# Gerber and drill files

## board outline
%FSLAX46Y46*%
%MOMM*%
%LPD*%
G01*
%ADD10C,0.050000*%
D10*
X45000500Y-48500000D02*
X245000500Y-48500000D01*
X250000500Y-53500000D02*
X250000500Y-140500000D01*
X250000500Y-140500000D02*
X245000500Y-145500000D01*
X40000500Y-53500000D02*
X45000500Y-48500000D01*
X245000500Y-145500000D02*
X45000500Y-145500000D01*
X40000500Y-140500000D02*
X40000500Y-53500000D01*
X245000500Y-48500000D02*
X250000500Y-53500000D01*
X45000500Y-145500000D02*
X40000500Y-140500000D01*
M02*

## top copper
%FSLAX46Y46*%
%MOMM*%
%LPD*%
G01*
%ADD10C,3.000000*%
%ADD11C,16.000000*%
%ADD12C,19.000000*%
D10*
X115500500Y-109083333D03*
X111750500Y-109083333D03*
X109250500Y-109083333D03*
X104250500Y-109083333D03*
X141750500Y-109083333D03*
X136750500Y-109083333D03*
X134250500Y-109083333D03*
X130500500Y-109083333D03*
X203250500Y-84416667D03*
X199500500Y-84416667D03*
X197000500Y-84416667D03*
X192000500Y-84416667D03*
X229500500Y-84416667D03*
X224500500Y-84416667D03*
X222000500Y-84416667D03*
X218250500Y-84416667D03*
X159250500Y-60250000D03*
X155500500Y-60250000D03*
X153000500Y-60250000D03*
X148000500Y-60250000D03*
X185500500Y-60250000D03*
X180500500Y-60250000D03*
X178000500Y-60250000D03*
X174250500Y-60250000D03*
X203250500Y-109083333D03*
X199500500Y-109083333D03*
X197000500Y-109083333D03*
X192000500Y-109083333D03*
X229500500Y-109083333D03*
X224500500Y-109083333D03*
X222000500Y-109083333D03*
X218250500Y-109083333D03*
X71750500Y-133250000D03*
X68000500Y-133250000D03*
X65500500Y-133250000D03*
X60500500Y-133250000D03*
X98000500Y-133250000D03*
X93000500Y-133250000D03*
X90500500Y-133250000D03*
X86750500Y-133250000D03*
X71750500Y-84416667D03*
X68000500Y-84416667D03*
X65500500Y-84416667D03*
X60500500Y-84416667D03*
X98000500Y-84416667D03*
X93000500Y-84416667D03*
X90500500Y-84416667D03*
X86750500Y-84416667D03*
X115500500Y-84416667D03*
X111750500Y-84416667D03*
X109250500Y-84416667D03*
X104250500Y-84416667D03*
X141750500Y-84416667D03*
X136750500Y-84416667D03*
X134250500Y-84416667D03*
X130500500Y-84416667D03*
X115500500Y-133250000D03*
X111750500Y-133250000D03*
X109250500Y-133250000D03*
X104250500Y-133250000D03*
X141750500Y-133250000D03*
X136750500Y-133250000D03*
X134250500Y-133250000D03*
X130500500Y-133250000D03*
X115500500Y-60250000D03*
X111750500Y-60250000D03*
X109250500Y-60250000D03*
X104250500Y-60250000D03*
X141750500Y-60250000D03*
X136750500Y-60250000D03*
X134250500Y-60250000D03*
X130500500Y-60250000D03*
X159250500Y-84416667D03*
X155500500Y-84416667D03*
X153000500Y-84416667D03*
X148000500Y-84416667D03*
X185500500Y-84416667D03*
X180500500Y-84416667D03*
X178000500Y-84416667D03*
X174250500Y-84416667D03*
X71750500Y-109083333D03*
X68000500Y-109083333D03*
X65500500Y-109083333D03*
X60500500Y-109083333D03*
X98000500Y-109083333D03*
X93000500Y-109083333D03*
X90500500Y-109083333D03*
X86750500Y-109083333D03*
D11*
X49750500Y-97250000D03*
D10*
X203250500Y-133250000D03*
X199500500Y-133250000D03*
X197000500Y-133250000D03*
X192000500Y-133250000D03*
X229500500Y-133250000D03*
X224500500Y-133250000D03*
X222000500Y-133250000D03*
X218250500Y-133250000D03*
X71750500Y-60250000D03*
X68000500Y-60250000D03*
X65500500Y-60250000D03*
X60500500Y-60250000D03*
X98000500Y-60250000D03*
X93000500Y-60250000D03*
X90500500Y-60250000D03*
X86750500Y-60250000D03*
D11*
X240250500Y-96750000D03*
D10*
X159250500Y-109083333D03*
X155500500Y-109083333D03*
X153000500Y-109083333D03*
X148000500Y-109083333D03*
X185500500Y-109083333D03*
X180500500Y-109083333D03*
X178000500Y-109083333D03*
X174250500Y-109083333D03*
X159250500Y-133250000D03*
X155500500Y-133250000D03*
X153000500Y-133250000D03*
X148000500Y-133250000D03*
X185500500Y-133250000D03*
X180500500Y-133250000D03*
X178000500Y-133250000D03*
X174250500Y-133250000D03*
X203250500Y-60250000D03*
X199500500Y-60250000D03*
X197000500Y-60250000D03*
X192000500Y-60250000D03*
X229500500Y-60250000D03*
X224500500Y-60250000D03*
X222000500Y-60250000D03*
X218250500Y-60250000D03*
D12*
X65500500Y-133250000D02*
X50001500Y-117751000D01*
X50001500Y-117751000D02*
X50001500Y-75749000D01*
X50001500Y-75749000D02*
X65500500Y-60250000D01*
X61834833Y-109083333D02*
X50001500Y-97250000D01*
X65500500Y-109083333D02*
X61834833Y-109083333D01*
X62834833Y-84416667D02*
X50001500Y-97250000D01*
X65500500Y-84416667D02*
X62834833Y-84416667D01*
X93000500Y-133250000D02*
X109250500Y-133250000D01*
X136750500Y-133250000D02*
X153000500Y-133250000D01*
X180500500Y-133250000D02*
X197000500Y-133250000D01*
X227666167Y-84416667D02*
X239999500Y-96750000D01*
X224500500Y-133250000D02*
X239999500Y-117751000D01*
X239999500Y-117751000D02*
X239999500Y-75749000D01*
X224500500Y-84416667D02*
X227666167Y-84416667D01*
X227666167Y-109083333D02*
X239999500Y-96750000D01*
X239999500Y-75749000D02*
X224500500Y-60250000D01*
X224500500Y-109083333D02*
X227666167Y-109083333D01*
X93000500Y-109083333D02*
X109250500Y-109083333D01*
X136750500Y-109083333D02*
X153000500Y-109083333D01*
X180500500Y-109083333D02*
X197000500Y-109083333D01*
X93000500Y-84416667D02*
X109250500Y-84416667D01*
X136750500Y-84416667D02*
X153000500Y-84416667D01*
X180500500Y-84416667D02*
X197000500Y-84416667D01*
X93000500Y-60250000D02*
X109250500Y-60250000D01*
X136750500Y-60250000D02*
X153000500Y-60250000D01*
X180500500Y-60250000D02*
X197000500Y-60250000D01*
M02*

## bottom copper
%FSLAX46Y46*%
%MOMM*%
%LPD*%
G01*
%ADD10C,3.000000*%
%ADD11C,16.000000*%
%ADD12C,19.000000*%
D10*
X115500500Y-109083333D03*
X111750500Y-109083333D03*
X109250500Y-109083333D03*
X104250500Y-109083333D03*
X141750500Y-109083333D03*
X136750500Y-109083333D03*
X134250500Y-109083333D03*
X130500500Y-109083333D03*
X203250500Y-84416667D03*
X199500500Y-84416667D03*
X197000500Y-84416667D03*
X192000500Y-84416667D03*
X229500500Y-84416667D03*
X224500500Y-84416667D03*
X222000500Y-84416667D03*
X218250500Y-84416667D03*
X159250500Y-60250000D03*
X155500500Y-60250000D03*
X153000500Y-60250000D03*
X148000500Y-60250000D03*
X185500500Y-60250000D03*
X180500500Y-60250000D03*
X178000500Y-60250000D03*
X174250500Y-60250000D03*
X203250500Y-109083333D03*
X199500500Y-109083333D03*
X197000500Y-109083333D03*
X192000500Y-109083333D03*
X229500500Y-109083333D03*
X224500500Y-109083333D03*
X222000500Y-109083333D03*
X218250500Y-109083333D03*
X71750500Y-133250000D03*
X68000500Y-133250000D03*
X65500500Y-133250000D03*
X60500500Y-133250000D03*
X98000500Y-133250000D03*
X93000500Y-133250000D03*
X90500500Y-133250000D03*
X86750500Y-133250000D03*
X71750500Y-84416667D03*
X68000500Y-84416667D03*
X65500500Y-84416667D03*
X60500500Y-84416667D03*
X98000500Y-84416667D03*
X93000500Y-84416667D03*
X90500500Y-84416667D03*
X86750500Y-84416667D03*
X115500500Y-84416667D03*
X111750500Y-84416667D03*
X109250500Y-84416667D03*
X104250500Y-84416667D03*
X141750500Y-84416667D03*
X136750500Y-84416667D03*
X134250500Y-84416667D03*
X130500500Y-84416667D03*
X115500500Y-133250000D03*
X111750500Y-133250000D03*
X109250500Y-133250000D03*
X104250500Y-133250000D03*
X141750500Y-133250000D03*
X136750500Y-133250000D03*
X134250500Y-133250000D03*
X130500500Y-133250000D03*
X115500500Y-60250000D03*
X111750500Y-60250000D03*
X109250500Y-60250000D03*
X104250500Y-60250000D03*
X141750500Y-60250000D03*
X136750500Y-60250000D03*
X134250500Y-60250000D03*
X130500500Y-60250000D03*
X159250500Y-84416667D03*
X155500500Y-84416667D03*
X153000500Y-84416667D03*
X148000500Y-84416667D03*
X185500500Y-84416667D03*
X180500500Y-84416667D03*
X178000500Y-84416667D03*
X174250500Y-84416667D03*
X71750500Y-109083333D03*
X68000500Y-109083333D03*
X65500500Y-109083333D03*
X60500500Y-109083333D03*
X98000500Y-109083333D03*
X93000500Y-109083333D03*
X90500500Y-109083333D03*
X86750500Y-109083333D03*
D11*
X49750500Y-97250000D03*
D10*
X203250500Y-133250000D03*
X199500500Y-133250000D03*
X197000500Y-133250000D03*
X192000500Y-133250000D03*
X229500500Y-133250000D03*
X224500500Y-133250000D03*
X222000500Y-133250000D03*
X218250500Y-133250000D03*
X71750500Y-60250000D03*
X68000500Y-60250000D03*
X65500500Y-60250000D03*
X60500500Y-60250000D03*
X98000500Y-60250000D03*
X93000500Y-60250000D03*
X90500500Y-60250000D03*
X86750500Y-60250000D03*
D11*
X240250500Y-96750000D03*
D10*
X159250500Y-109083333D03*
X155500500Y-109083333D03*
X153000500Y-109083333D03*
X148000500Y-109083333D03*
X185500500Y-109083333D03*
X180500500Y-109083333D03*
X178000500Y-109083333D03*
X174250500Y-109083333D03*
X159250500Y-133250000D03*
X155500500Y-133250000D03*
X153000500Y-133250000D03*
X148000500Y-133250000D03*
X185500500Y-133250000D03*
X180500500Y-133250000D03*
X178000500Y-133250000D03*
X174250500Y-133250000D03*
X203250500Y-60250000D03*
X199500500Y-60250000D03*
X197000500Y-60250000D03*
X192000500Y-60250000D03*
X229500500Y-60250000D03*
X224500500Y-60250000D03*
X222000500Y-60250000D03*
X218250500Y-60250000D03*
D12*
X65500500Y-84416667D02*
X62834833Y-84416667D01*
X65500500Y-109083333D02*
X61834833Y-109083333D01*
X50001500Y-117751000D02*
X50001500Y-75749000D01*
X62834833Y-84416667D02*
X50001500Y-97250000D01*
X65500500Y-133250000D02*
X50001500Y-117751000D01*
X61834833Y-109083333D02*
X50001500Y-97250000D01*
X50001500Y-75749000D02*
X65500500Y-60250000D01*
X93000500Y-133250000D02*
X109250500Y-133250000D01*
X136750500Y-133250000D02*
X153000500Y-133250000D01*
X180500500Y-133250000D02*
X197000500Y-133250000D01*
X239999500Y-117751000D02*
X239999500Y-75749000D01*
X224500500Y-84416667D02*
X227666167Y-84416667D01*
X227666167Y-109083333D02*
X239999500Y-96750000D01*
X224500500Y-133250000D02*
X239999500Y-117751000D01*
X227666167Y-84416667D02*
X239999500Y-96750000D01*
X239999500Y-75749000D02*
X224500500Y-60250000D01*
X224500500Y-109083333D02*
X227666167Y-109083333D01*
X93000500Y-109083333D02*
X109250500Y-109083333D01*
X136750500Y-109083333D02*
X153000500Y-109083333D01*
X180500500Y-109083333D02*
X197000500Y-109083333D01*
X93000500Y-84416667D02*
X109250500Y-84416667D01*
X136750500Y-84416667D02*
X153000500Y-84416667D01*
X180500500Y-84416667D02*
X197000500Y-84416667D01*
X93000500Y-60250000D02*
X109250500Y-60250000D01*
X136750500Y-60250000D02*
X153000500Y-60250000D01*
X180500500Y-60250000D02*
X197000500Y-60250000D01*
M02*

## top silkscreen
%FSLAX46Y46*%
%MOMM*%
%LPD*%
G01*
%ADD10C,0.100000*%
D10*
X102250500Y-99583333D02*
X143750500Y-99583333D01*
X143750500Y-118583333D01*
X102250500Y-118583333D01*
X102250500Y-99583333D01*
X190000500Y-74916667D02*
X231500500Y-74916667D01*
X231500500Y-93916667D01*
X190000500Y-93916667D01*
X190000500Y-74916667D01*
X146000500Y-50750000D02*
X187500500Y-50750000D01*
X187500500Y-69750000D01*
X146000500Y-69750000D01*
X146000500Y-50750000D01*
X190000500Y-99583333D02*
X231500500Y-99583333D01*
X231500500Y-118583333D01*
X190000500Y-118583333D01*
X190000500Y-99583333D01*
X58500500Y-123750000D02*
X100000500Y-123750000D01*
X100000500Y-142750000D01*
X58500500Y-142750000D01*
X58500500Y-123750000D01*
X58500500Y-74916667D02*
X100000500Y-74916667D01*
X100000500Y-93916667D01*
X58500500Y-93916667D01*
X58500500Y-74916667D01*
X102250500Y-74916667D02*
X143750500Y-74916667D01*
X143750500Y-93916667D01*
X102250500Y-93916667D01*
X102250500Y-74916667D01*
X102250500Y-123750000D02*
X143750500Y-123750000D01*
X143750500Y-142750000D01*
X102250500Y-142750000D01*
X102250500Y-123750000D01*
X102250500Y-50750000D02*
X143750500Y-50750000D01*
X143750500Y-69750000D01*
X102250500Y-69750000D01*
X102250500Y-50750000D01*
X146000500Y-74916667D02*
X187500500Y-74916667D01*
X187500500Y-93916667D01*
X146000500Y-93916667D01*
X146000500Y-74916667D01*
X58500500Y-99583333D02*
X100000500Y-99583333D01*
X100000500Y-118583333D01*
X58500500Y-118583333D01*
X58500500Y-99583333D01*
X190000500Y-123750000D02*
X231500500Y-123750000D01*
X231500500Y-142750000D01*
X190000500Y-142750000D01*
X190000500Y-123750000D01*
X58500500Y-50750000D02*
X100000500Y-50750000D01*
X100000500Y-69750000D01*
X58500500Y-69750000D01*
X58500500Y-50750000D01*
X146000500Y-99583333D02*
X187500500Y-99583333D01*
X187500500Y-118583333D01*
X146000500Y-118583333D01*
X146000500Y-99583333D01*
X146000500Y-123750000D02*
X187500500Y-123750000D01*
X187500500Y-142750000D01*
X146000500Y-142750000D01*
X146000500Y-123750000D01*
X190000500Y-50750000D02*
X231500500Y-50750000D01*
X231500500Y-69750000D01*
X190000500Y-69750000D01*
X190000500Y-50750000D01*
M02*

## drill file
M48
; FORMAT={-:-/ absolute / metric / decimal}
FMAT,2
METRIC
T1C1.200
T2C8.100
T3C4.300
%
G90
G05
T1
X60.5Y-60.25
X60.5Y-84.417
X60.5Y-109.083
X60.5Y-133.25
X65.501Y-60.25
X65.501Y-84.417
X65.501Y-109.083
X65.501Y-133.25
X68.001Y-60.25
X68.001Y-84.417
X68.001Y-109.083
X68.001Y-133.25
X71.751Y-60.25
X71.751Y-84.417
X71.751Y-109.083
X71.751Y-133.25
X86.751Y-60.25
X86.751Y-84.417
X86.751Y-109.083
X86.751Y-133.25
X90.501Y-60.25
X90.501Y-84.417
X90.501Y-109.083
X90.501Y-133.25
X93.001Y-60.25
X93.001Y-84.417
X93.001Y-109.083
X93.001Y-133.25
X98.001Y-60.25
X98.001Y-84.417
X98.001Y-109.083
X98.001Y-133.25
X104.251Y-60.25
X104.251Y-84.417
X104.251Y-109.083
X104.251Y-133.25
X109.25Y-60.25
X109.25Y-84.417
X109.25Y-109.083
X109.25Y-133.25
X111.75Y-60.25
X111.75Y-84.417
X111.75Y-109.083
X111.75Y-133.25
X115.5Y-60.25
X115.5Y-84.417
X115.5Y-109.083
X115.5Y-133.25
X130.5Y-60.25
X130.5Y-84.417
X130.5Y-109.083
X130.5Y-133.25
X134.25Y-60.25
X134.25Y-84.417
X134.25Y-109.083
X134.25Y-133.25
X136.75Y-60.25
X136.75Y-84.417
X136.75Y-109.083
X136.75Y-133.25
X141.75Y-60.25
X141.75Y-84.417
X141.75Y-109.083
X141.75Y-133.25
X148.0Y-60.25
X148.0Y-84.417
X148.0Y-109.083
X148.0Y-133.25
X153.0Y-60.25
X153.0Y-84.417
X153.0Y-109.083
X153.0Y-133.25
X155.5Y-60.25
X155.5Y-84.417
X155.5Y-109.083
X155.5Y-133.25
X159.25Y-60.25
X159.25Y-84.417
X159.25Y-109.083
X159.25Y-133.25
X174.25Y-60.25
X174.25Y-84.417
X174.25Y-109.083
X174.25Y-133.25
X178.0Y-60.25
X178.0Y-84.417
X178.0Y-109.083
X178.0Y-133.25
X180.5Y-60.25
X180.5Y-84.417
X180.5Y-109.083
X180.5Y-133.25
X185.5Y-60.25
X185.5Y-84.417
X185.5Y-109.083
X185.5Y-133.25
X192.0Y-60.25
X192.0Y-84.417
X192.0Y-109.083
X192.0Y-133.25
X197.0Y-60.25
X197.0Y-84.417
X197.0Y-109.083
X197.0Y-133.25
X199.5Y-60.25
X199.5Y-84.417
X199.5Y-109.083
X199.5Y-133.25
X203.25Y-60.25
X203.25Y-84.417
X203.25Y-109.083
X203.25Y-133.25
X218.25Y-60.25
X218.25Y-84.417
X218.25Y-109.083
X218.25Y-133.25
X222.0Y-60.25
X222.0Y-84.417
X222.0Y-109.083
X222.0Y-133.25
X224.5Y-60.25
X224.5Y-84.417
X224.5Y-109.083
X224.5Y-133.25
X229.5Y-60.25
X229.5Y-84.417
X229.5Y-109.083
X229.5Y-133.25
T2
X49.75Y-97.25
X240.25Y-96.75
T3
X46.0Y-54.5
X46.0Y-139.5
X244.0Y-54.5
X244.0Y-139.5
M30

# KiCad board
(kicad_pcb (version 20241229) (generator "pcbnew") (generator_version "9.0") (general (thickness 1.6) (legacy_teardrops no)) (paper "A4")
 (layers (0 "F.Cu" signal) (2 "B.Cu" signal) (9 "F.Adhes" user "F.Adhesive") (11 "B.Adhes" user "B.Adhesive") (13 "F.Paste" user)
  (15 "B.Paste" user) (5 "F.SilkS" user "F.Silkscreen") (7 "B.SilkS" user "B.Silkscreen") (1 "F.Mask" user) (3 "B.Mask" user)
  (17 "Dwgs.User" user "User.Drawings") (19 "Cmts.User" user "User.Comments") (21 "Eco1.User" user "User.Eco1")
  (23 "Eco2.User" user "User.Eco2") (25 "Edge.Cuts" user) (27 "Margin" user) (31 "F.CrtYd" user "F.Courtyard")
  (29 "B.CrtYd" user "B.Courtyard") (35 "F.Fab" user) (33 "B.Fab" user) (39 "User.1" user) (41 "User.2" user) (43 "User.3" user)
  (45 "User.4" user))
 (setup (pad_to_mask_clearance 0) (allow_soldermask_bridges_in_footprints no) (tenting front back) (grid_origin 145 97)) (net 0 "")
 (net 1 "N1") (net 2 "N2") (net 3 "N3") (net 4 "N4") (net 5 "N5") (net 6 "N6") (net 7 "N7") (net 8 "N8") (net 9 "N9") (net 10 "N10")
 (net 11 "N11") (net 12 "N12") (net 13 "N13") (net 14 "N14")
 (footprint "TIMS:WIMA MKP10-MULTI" (layer "F.Cu") (at 123.0005 109.083333 -90)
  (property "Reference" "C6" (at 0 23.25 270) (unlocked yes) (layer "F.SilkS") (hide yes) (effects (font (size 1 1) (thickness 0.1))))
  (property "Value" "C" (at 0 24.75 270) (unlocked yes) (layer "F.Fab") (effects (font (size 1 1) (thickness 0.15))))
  (fp_rect (start -9.5 -20.75) (end 9.5 20.75) (stroke (width 0.1) (type solid)) (fill no) (layer "F.SilkS"))
  (pad "1" thru_hole circle (at 0 7.5 270) (size 3 3) (drill 1.2) (layers "*.Cu" "*.Mask") (remove_unused_layers no) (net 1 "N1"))
  (pad "1" thru_hole circle (at 0 11.25 270) (size 3 3) (drill 1.2) (layers "*.Cu" "*.Mask") (remove_unused_layers no) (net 1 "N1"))
  (pad "1" thru_hole circle (at 0 13.75 270) (size 3 3) (drill 1.2) (layers "*.Cu" "*.Mask") (remove_unused_layers no) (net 1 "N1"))
  (pad "1" thru_hole circle (at 0 18.75 270) (size 3 3) (drill 1.2) (layers "*.Cu" "*.Mask") (remove_unused_layers no) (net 1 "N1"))
  (pad "2" thru_hole circle (at 0 -18.75 270) (size 3 3) (drill 1.2) (layers "*.Cu" "*.Mask") (remove_unused_layers no) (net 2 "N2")
   (zone_connect 2))
  (pad "2" thru_hole circle (at 0 -13.75 270) (size 3 3) (drill 1.2) (layers "*.Cu" "*.Mask") (remove_unused_layers no) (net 2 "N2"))
  (pad "2" thru_hole circle (at 0 -11.25 270) (size 3 3) (drill 1.2) (layers "*.Cu" "*.Mask") (remove_unused_layers no) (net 2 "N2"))
  (pad "2" thru_hole circle (at 0 -7.5 270) (size 3 3) (drill 1.2) (layers "*.Cu" "*.Mask") (remove_unused_layers no) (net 2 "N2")))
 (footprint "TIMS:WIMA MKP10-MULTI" (layer "F.Cu") (at 210.7505 84.416667 -90)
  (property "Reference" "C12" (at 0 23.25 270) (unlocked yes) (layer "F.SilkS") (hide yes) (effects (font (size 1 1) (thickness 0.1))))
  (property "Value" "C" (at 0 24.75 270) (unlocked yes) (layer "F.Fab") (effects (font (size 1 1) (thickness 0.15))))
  (fp_rect (start -9.5 -20.75) (end 9.5 20.75) (stroke (width 0.1) (type solid)) (fill no) (layer "F.SilkS"))
  (pad "1" thru_hole circle (at 0 7.5 270) (size 3 3) (drill 1.2) (layers "*.Cu" "*.Mask") (remove_unused_layers no) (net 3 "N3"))
  (pad "1" thru_hole circle (at 0 11.25 270) (size 3 3) (drill 1.2) (layers "*.Cu" "*.Mask") (remove_unused_layers no) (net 3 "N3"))
  (pad "1" thru_hole circle (at 0 13.75 270) (size 3 3) (drill 1.2) (layers "*.Cu" "*.Mask") (remove_unused_layers no) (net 3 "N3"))
  (pad "1" thru_hole circle (at 0 18.75 270) (size 3 3) (drill 1.2) (layers "*.Cu" "*.Mask") (remove_unused_layers no) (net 3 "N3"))
  (pad "2" thru_hole circle (at 0 -18.75 270) (size 3 3) (drill 1.2) (layers "*.Cu" "*.Mask") (remove_unused_layers no) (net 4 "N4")
   (zone_connect 2))
  (pad "2" thru_hole circle (at 0 -13.75 270) (size 3 3) (drill 1.2) (layers "*.Cu" "*.Mask") (remove_unused_layers no) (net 4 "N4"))
  (pad "2" thru_hole circle (at 0 -11.25 270) (size 3 3) (drill 1.2) (layers "*.Cu" "*.Mask") (remove_unused_layers no) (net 4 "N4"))
  (pad "2" thru_hole circle (at 0 -7.5 270) (size 3 3) (drill 1.2) (layers "*.Cu" "*.Mask") (remove_unused_layers no) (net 4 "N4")))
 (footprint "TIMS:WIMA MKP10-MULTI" (layer "F.Cu") (at 166.7505 60.25 -90)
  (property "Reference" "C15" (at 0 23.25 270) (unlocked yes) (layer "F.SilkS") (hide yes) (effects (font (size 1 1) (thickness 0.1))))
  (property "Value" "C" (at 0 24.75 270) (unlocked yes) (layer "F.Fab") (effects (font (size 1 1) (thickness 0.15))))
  (fp_rect (start -9.5 -20.75) (end 9.5 20.75) (stroke (width 0.1) (type solid)) (fill no) (layer "F.SilkS"))
  (pad "1" thru_hole circle (at 0 7.5 270) (size 3 3) (drill 1.2) (layers "*.Cu" "*.Mask") (remove_unused_layers no) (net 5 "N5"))
  (pad "1" thru_hole circle (at 0 11.25 270) (size 3 3) (drill 1.2) (layers "*.Cu" "*.Mask") (remove_unused_layers no) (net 5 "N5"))
  (pad "1" thru_hole circle (at 0 13.75 270) (size 3 3) (drill 1.2) (layers "*.Cu" "*.Mask") (remove_unused_layers no) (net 5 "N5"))
  (pad "1" thru_hole circle (at 0 18.75 270) (size 3 3) (drill 1.2) (layers "*.Cu" "*.Mask") (remove_unused_layers no) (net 5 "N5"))
  (pad "2" thru_hole circle (at 0 -18.75 270) (size 3 3) (drill 1.2) (layers "*.Cu" "*.Mask") (remove_unused_layers no) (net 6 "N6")
   (zone_connect 2))
  (pad "2" thru_hole circle (at 0 -13.75 270) (size 3 3) (drill 1.2) (layers "*.Cu" "*.Mask") (remove_unused_layers no) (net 6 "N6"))
  (pad "2" thru_hole circle (at 0 -11.25 270) (size 3 3) (drill 1.2) (layers "*.Cu" "*.Mask") (remove_unused_layers no) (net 6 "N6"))
  (pad "2" thru_hole circle (at 0 -7.5 270) (size 3 3) (drill 1.2) (layers "*.Cu" "*.Mask") (remove_unused_layers no) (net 6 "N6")))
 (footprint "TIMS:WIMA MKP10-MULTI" (layer "F.Cu") (at 210.7505 109.083333 -90)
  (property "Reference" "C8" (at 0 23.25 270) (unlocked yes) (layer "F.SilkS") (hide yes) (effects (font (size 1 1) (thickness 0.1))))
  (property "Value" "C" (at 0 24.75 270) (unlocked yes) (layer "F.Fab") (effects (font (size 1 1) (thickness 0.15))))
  (fp_rect (start -9.5 -20.75) (end 9.5 20.75) (stroke (width 0.1) (type solid)) (fill no) (layer "F.SilkS"))
  (pad "1" thru_hole circle (at 0 7.5 270) (size 3 3) (drill 1.2) (layers "*.Cu" "*.Mask") (remove_unused_layers no) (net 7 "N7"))
  (pad "1" thru_hole circle (at 0 11.25 270) (size 3 3) (drill 1.2) (layers "*.Cu" "*.Mask") (remove_unused_layers no) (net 7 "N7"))
  (pad "1" thru_hole circle (at 0 13.75 270) (size 3 3) (drill 1.2) (layers "*.Cu" "*.Mask") (remove_unused_layers no) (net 7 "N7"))
  (pad "1" thru_hole circle (at 0 18.75 270) (size 3 3) (drill 1.2) (layers "*.Cu" "*.Mask") (remove_unused_layers no) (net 7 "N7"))
  (pad "2" thru_hole circle (at 0 -18.75 270) (size 3 3) (drill 1.2) (layers "*.Cu" "*.Mask") (remove_unused_layers no) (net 4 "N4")
   (zone_connect 2))
  (pad "2" thru_hole circle (at 0 -13.75 270) (size 3 3) (drill 1.2) (layers "*.Cu" "*.Mask") (remove_unused_layers no) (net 4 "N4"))
  (pad "2" thru_hole circle (at 0 -11.25 270) (size 3 3) (drill 1.2) (layers "*.Cu" "*.Mask") (remove_unused_layers no) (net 4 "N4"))
  (pad "2" thru_hole circle (at 0 -7.5 270) (size 3 3) (drill 1.2) (layers "*.Cu" "*.Mask") (remove_unused_layers no) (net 4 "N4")))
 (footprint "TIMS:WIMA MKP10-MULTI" (layer "F.Cu") (at 79.2505 133.25 -90)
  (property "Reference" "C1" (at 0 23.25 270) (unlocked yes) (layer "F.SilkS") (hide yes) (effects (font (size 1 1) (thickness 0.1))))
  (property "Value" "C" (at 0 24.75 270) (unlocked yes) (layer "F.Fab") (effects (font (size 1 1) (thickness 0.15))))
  (fp_rect (start -9.5 -20.75) (end 9.5 20.75) (stroke (width 0.1) (type solid)) (fill no) (layer "F.SilkS"))
  (pad "1" thru_hole circle (at 0 7.5 270) (size 3 3) (drill 1.2) (layers "*.Cu" "*.Mask") (remove_unused_layers no) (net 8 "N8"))
  (pad "1" thru_hole circle (at 0 11.25 270) (size 3 3) (drill 1.2) (layers "*.Cu" "*.Mask") (remove_unused_layers no) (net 8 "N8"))
  (pad "1" thru_hole circle (at 0 13.75 270) (size 3 3) (drill 1.2) (layers "*.Cu" "*.Mask") (remove_unused_layers no) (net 8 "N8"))
  (pad "1" thru_hole circle (at 0 18.75 270) (size 3 3) (drill 1.2) (layers "*.Cu" "*.Mask") (remove_unused_layers no) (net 8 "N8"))
  (pad "2" thru_hole circle (at 0 -18.75 270) (size 3 3) (drill 1.2) (layers "*.Cu" "*.Mask") (remove_unused_layers no) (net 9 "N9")
   (zone_connect 2))
  (pad "2" thru_hole circle (at 0 -13.75 270) (size 3 3) (drill 1.2) (layers "*.Cu" "*.Mask") (remove_unused_layers no) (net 9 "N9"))
  (pad "2" thru_hole circle (at 0 -11.25 270) (size 3 3) (drill 1.2) (layers "*.Cu" "*.Mask") (remove_unused_layers no) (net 9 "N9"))
  (pad "2" thru_hole circle (at 0 -7.5 270) (size 3 3) (drill 1.2) (layers "*.Cu" "*.Mask") (remove_unused_layers no) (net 9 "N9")))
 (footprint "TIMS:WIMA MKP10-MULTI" (layer "F.Cu") (at 79.2505 84.416667 -90)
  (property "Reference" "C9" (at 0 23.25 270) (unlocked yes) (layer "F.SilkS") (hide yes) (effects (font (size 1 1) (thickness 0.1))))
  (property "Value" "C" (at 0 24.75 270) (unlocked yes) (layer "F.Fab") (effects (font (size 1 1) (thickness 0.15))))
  (fp_rect (start -9.5 -20.75) (end 9.5 20.75) (stroke (width 0.1) (type solid)) (fill no) (layer "F.SilkS"))
  (pad "1" thru_hole circle (at 0 7.5 270) (size 3 3) (drill 1.2) (layers "*.Cu" "*.Mask") (remove_unused_layers no) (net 8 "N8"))
  (pad "1" thru_hole circle (at 0 11.25 270) (size 3 3) (drill 1.2) (layers "*.Cu" "*.Mask") (remove_unused_layers no) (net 8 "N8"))
  (pad "1" thru_hole circle (at 0 13.75 270) (size 3 3) (drill 1.2) (layers "*.Cu" "*.Mask") (remove_unused_layers no) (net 8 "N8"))
  (pad "1" thru_hole circle (at 0 18.75 270) (size 3 3) (drill 1.2) (layers "*.Cu" "*.Mask") (remove_unused_layers no) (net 8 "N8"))
  (pad "2" thru_hole circle (at 0 -18.75 270) (size 3 3) (drill 1.2) (layers "*.Cu" "*.Mask") (remove_unused_layers no) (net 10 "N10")
   (zone_connect 2))
  (pad "2" thru_hole circle (at 0 -13.75 270) (size 3 3) (drill 1.2) (layers "*.Cu" "*.Mask") (remove_unused_layers no) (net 10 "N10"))
  (pad "2" thru_hole circle (at 0 -11.25 270) (size 3 3) (drill 1.2) (layers "*.Cu" "*.Mask") (remove_unused_layers no) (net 10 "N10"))
  (pad "2" thru_hole circle (at 0 -7.5 270) (size 3 3) (drill 1.2) (layers "*.Cu" "*.Mask") (remove_unused_layers no) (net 10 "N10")))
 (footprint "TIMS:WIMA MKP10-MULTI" (layer "F.Cu") (at 123.0005 84.416667 -90)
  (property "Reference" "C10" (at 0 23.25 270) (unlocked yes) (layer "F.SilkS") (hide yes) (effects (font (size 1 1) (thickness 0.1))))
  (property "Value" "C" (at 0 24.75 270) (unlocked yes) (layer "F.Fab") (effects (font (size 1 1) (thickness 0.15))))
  (fp_rect (start -9.5 -20.75) (end 9.5 20.75) (stroke (width 0.1) (type solid)) (fill no) (layer "F.SilkS"))
  (pad "1" thru_hole circle (at 0 7.5 270) (size 3 3) (drill 1.2) (layers "*.Cu" "*.Mask") (remove_unused_layers no) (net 10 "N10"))
  (pad "1" thru_hole circle (at 0 11.25 270) (size 3 3) (drill 1.2) (layers "*.Cu" "*.Mask") (remove_unused_layers no) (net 10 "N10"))
  (pad "1" thru_hole circle (at 0 13.75 270) (size 3 3) (drill 1.2) (layers "*.Cu" "*.Mask") (remove_unused_layers no) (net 10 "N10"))
  (pad "1" thru_hole circle (at 0 18.75 270) (size 3 3) (drill 1.2) (layers "*.Cu" "*.Mask") (remove_unused_layers no) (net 10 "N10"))
  (pad "2" thru_hole circle (at 0 -18.75 270) (size 3 3) (drill 1.2) (layers "*.Cu" "*.Mask") (remove_unused_layers no) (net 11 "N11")
   (zone_connect 2))
  (pad "2" thru_hole circle (at 0 -13.75 270) (size 3 3) (drill 1.2) (layers "*.Cu" "*.Mask") (remove_unused_layers no) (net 11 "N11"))
  (pad "2" thru_hole circle (at 0 -11.25 270) (size 3 3) (drill 1.2) (layers "*.Cu" "*.Mask") (remove_unused_layers no) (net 11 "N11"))
  (pad "2" thru_hole circle (at 0 -7.5 270) (size 3 3) (drill 1.2) (layers "*.Cu" "*.Mask") (remove_unused_layers no) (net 11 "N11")))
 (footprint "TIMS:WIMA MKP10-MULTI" (layer "F.Cu") (at 123.0005 133.25 -90)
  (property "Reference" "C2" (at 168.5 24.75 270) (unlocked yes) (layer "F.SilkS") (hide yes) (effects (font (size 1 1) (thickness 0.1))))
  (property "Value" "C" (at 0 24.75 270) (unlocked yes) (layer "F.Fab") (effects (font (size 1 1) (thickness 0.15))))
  (fp_rect (start -9.5 -20.75) (end 9.5 20.75) (stroke (width 0.1) (type solid)) (fill no) (layer "F.SilkS"))
  (pad "1" thru_hole circle (at 0 7.5 270) (size 3 3) (drill 1.2) (layers "*.Cu" "*.Mask") (remove_unused_layers no) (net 9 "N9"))
  (pad "1" thru_hole circle (at 0 11.25 270) (size 3 3) (drill 1.2) (layers "*.Cu" "*.Mask") (remove_unused_layers no) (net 9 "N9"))
  (pad "1" thru_hole circle (at 0 13.75 270) (size 3 3) (drill 1.2) (layers "*.Cu" "*.Mask") (remove_unused_layers no) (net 9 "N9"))
  (pad "1" thru_hole circle (at 0 18.75 270) (size 3 3) (drill 1.2) (layers "*.Cu" "*.Mask") (remove_unused_layers no) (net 9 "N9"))
  (pad "2" thru_hole circle (at 0 -18.75 270) (size 3 3) (drill 1.2) (layers "*.Cu" "*.Mask") (remove_unused_layers no) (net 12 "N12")
   (zone_connect 2))
  (pad "2" thru_hole circle (at 0 -13.75 270) (size 3 3) (drill 1.2) (layers "*.Cu" "*.Mask") (remove_unused_layers no) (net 12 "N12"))
  (pad "2" thru_hole circle (at 0 -11.25 270) (size 3 3) (drill 1.2) (layers "*.Cu" "*.Mask") (remove_unused_layers no) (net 12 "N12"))
  (pad "2" thru_hole circle (at 0 -7.5 270) (size 3 3) (drill 1.2) (layers "*.Cu" "*.Mask") (remove_unused_layers no) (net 12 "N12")))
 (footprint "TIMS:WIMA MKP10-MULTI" (layer "F.Cu") (at 123.0005 60.25 -90)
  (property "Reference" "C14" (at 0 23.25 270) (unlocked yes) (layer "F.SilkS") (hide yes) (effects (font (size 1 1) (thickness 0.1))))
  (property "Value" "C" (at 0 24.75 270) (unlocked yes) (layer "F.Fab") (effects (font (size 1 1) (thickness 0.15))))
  (fp_rect (start -9.5 -20.75) (end 9.5 20.75) (stroke (width 0.1) (type solid)) (fill no) (layer "F.SilkS"))
  (pad "1" thru_hole circle (at 0 7.5 270) (size 3 3) (drill 1.2) (layers "*.Cu" "*.Mask") (remove_unused_layers no) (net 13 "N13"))
  (pad "1" thru_hole circle (at 0 11.25 270) (size 3 3) (drill 1.2) (layers "*.Cu" "*.Mask") (remove_unused_layers no) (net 13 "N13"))
  (pad "1" thru_hole circle (at 0 13.75 270) (size 3 3) (drill 1.2) (layers "*.Cu" "*.Mask") (remove_unused_layers no) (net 13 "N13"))
  (pad "1" thru_hole circle (at 0 18.75 270) (size 3 3) (drill 1.2) (layers "*.Cu" "*.Mask") (remove_unused_layers no) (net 13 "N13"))
  (pad "2" thru_hole circle (at 0 -18.75 270) (size 3 3) (drill 1.2) (layers "*.Cu" "*.Mask") (remove_unused_layers no) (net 5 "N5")
   (zone_connect 2))
  (pad "2" thru_hole circle (at 0 -13.75 270) (size 3 3) (drill 1.2) (layers "*.Cu" "*.Mask") (remove_unused_layers no) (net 5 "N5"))
  (pad "2" thru_hole circle (at 0 -11.25 270) (size 3 3) (drill 1.2) (layers "*.Cu" "*.Mask") (remove_unused_layers no) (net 5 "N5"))
  (pad "2" thru_hole circle (at 0 -7.5 270) (size 3 3) (drill 1.2) (layers "*.Cu" "*.Mask") (remove_unused_layers no) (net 5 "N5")))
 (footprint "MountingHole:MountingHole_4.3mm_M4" (layer "F.Cu") (at 46 54.5)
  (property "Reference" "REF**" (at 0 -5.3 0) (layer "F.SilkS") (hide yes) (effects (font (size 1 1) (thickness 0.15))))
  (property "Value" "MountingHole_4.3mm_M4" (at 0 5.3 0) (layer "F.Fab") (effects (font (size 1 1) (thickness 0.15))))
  (pad "" np_thru_hole circle (at 0 0) (size 4.3 4.3) (drill 4.3) (layers "*.Cu" "*.Mask")))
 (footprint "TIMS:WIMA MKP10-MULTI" (layer "F.Cu") (at 166.7505 84.416667 -90)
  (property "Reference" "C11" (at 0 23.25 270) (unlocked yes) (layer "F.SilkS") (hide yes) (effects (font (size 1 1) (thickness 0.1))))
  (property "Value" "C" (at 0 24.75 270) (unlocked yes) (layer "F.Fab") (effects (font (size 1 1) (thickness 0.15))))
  (fp_rect (start -9.5 -20.75) (end 9.5 20.75) (stroke (width 0.1) (type solid)) (fill no) (layer "F.SilkS"))
  (pad "1" thru_hole circle (at 0 7.5 270) (size 3 3) (drill 1.2) (layers "*.Cu" "*.Mask") (remove_unused_layers no) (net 11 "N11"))
  (pad "1" thru_hole circle (at 0 11.25 270) (size 3 3) (drill 1.2) (layers "*.Cu" "*.Mask") (remove_unused_layers no) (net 11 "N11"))
  (pad "1" thru_hole circle (at 0 13.75 270) (size 3 3) (drill 1.2) (layers "*.Cu" "*.Mask") (remove_unused_layers no) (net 11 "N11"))
  (pad "1" thru_hole circle (at 0 18.75 270) (size 3 3) (drill 1.2) (layers "*.Cu" "*.Mask") (remove_unused_layers no) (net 11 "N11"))
  (pad "2" thru_hole circle (at 0 -18.75 270) (size 3 3) (drill 1.2) (layers "*.Cu" "*.Mask") (remove_unused_layers no) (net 3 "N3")
   (zone_connect 2))
  (pad "2" thru_hole circle (at 0 -13.75 270) (size 3 3) (drill 1.2) (layers "*.Cu" "*.Mask") (remove_unused_layers no) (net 3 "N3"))
  (pad "2" thru_hole circle (at 0 -11.25 270) (size 3 3) (drill 1.2) (layers "*.Cu" "*.Mask") (remove_unused_layers no) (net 3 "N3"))
  (pad "2" thru_hole circle (at 0 -7.5 270) (size 3 3) (drill 1.2) (layers "*.Cu" "*.Mask") (remove_unused_layers no) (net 3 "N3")))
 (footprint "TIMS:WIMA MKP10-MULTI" (layer "F.Cu") (at 79.2505 109.083333 -90)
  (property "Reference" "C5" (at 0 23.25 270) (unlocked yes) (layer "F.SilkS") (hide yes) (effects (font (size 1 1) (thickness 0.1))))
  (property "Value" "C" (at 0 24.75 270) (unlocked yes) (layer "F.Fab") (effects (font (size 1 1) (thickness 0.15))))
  (fp_rect (start -9.5 -20.75) (end 9.5 20.75) (stroke (width 0.1) (type solid)) (fill no) (layer "F.SilkS"))
  (pad "1" thru_hole circle (at 0 7.5 270) (size 3 3) (drill 1.2) (layers "*.Cu" "*.Mask") (remove_unused_layers no) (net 8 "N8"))
  (pad "1" thru_hole circle (at 0 11.25 270) (size 3 3) (drill 1.2) (layers "*.Cu" "*.Mask") (remove_unused_layers no) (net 8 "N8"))
  (pad "1" thru_hole circle (at 0 13.75 270) (size 3 3) (drill 1.2) (layers "*.Cu" "*.Mask") (remove_unused_layers no) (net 8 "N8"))
  (pad "1" thru_hole circle (at 0 18.75 270) (size 3 3) (drill 1.2) (layers "*.Cu" "*.Mask") (remove_unused_layers no) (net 8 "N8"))
  (pad "2" thru_hole circle (at 0 -18.75 270) (size 3 3) (drill 1.2) (layers "*.Cu" "*.Mask") (remove_unused_layers no) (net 1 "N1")
   (zone_connect 2))
  (pad "2" thru_hole circle (at 0 -13.75 270) (size 3 3) (drill 1.2) (layers "*.Cu" "*.Mask") (remove_unused_layers no) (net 1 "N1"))
  (pad "2" thru_hole circle (at 0 -11.25 270) (size 3 3) (drill 1.2) (layers "*.Cu" "*.Mask") (remove_unused_layers no) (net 1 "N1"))
  (pad "2" thru_hole circle (at 0 -7.5 270) (size 3 3) (drill 1.2) (layers "*.Cu" "*.Mask") (remove_unused_layers no) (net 1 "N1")))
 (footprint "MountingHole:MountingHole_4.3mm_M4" (layer "F.Cu") (at 244 139.5)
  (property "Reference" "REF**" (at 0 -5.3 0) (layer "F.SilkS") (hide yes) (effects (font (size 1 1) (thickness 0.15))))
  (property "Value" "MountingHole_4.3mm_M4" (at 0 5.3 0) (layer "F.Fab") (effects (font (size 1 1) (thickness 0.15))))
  (pad "" np_thru_hole circle (at 0 0) (size 4.3 4.3) (drill 4.3) (layers "*.Cu" "*.Mask")))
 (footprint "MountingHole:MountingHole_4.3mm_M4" (layer "F.Cu") (at 244 54.5)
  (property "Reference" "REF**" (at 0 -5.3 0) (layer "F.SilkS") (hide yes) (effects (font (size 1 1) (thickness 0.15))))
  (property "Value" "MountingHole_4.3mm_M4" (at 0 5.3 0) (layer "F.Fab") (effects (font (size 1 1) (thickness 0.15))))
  (pad "" np_thru_hole circle (at 0 0) (size 4.3 4.3) (drill 4.3) (layers "*.Cu" "*.Mask")))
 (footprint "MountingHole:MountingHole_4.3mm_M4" (layer "F.Cu") (at 46 139.5)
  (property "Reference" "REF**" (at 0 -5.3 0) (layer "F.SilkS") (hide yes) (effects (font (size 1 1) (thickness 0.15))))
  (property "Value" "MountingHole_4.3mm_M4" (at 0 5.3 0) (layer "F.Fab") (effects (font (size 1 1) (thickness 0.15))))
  (pad "" np_thru_hole circle (at 0 0) (size 4.3 4.3) (drill 4.3) (layers "*.Cu" "*.Mask")))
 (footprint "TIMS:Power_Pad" (layer "F.Cu") (at 49.7505 97.25)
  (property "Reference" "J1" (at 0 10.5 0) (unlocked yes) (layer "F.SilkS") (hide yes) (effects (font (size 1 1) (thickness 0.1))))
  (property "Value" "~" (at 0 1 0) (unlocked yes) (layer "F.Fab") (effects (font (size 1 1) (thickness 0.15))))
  (pad "1" thru_hole circle (at 0 0) (size 16 16) (drill 8.1) (layers "*.Cu" "*.Mask") (remove_unused_layers no) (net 8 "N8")))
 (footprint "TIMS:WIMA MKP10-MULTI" (layer "F.Cu") (at 210.7505 133.25 -90)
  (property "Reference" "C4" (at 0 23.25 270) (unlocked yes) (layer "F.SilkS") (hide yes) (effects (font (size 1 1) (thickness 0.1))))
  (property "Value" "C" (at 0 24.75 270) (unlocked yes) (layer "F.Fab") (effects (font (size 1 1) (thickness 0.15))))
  (fp_rect (start -9.5 -20.75) (end 9.5 20.75) (stroke (width 0.1) (type solid)) (fill no) (layer "F.SilkS"))
  (pad "1" thru_hole circle (at 0 7.5 270) (size 3 3) (drill 1.2) (layers "*.Cu" "*.Mask") (remove_unused_layers no) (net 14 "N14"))
  (pad "1" thru_hole circle (at 0 11.25 270) (size 3 3) (drill 1.2) (layers "*.Cu" "*.Mask") (remove_unused_layers no) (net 14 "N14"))
  (pad "1" thru_hole circle (at 0 13.75 270) (size 3 3) (drill 1.2) (layers "*.Cu" "*.Mask") (remove_unused_layers no) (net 14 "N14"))
  (pad "1" thru_hole circle (at 0 18.75 270) (size 3 3) (drill 1.2) (layers "*.Cu" "*.Mask") (remove_unused_layers no) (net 14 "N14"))
  (pad "2" thru_hole circle (at 0 -18.75 270) (size 3 3) (drill 1.2) (layers "*.Cu" "*.Mask") (remove_unused_layers no) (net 4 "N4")
   (zone_connect 2))
  (pad "2" thru_hole circle (at 0 -13.75 270) (size 3 3) (drill 1.2) (layers "*.Cu" "*.Mask") (remove_unused_layers no) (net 4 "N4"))
  (pad "2" thru_hole circle (at 0 -11.25 270) (size 3 3) (drill 1.2) (layers "*.Cu" "*.Mask") (remove_unused_layers no) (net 4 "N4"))
  (pad "2" thru_hole circle (at 0 -7.5 270) (size 3 3) (drill 1.2) (layers "*.Cu" "*.Mask") (remove_unused_layers no) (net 4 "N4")))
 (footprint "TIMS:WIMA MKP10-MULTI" (layer "F.Cu") (at 79.2505 60.25 -90)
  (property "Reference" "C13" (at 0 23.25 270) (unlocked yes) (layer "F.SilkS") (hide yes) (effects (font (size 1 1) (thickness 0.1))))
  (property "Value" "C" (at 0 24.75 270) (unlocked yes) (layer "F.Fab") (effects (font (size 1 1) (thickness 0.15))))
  (fp_rect (start -9.5 -20.75) (end 9.5 20.75) (stroke (width 0.1) (type solid)) (fill no) (layer "F.SilkS"))
  (pad "1" thru_hole circle (at 0 7.5 270) (size 3 3) (drill 1.2) (layers "*.Cu" "*.Mask") (remove_unused_layers no) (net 8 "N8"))
  (pad "1" thru_hole circle (at 0 11.25 270) (size 3 3) (drill 1.2) (layers "*.Cu" "*.Mask") (remove_unused_layers no) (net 8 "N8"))
  (pad "1" thru_hole circle (at 0 13.75 270) (size 3 3) (drill 1.2) (layers "*.Cu" "*.Mask") (remove_unused_layers no) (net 8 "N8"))
  (pad "1" thru_hole circle (at 0 18.75 270) (size 3 3) (drill 1.2) (layers "*.Cu" "*.Mask") (remove_unused_layers no) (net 8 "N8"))
  (pad "2" thru_hole circle (at 0 -18.75 270) (size 3 3) (drill 1.2) (layers "*.Cu" "*.Mask") (remove_unused_layers no) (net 13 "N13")
   (zone_connect 2))
  (pad "2" thru_hole circle (at 0 -13.75 270) (size 3 3) (drill 1.2) (layers "*.Cu" "*.Mask") (remove_unused_layers no) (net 13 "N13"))
  (pad "2" thru_hole circle (at 0 -11.25 270) (size 3 3) (drill 1.2) (layers "*.Cu" "*.Mask") (remove_unused_layers no) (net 13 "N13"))
  (pad "2" thru_hole circle (at 0 -7.5 270) (size 3 3) (drill 1.2) (layers "*.Cu" "*.Mask") (remove_unused_layers no) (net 13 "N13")))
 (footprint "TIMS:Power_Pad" (layer "F.Cu") (at 240.2505 96.75)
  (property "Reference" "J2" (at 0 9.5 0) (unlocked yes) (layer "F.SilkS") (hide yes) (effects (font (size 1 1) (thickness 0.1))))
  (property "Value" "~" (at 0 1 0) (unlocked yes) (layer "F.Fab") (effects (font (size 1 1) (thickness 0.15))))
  (pad "1" thru_hole circle (at 0 0) (size 16 16) (drill 8.1) (layers "*.Cu" "*.Mask") (remove_unused_layers no) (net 4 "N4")))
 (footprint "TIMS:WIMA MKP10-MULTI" (layer "F.Cu") (at 166.7505 109.083333 -90)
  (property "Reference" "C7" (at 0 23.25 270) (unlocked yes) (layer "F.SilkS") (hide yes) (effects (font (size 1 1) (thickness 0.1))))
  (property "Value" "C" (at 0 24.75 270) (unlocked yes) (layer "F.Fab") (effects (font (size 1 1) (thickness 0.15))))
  (fp_rect (start -9.5 -20.75) (end 9.5 20.75) (stroke (width 0.1) (type solid)) (fill no) (layer "F.SilkS"))
  (pad "1" thru_hole circle (at 0 7.5 270) (size 3 3) (drill 1.2) (layers "*.Cu" "*.Mask") (remove_unused_layers no) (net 2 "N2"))
  (pad "1" thru_hole circle (at 0 11.25 270) (size 3 3) (drill 1.2) (layers "*.Cu" "*.Mask") (remove_unused_layers no) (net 2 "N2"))
  (pad "1" thru_hole circle (at 0 13.75 270) (size 3 3) (drill 1.2) (layers "*.Cu" "*.Mask") (remove_unused_layers no) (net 2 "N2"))
  (pad "1" thru_hole circle (at 0 18.75 270) (size 3 3) (drill 1.2) (layers "*.Cu" "*.Mask") (remove_unused_layers no) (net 2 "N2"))
  (pad "2" thru_hole circle (at 0 -18.75 270) (size 3 3) (drill 1.2) (layers "*.Cu" "*.Mask") (remove_unused_layers no) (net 7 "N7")
   (zone_connect 2))
  (pad "2" thru_hole circle (at 0 -13.75 270) (size 3 3) (drill 1.2) (layers "*.Cu" "*.Mask") (remove_unused_layers no) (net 7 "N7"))
  (pad "2" thru_hole circle (at 0 -11.25 270) (size 3 3) (drill 1.2) (layers "*.Cu" "*.Mask") (remove_unused_layers no) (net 7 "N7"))
  (pad "2" thru_hole circle (at 0 -7.5 270) (size 3 3) (drill 1.2) (layers "*.Cu" "*.Mask") (remove_unused_layers no) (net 7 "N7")))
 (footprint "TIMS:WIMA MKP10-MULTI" (layer "F.Cu") (at 166.7505 133.25 -90)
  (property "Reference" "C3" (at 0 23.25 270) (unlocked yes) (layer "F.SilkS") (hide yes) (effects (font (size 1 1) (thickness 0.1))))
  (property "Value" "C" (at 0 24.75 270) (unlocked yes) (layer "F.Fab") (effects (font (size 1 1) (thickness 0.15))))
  (fp_rect (start -9.5 -20.75) (end 9.5 20.75) (stroke (width 0.1) (type solid)) (fill no) (layer "F.SilkS"))
  (pad "1" thru_hole circle (at 0 7.5 270) (size 3 3) (drill 1.2) (layers "*.Cu" "*.Mask") (remove_unused_layers no) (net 12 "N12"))
  (pad "1" thru_hole circle (at 0 11.25 270) (size 3 3) (drill 1.2) (layers "*.Cu" "*.Mask") (remove_unused_layers no) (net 12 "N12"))
  (pad "1" thru_hole circle (at 0 13.75 270) (size 3 3) (drill 1.2) (layers "*.Cu" "*.Mask") (remove_unused_layers no) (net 12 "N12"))
  (pad "1" thru_hole circle (at 0 18.75 270) (size 3 3) (drill 1.2) (layers "*.Cu" "*.Mask") (remove_unused_layers no) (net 12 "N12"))
  (pad "2" thru_hole circle (at 0 -18.75 270) (size 3 3) (drill 1.2) (layers "*.Cu" "*.Mask") (remove_unused_layers no) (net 14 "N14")
   (zone_connect 2))
  (pad "2" thru_hole circle (at 0 -13.75 270) (size 3 3) (drill 1.2) (layers "*.Cu" "*.Mask") (remove_unused_layers no) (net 14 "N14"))
  (pad "2" thru_hole circle (at 0 -11.25 270) (size 3 3) (drill 1.2) (layers "*.Cu" "*.Mask") (remove_unused_layers no) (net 14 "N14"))
  (pad "2" thru_hole circle (at 0 -7.5 270) (size 3 3) (drill 1.2) (layers "*.Cu" "*.Mask") (remove_unused_layers no) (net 14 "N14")))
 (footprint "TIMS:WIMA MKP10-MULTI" (layer "F.Cu") (at 210.7505 60.25 -90)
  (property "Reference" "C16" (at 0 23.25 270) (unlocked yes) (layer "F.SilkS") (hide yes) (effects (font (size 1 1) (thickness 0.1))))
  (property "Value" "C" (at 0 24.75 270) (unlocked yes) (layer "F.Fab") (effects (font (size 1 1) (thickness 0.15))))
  (fp_rect (start -9.5 -20.75) (end 9.5 20.75) (stroke (width 0.1) (type solid)) (fill no) (layer "F.SilkS"))
  (pad "1" thru_hole circle (at 0 7.5 270) (size 3 3) (drill 1.2) (layers "*.Cu" "*.Mask") (remove_unused_layers no) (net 6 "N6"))
  (pad "1" thru_hole circle (at 0 11.25 270) (size 3 3) (drill 1.2) (layers "*.Cu" "*.Mask") (remove_unused_layers no) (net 6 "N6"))
  (pad "1" thru_hole circle (at 0 13.75 270) (size 3 3) (drill 1.2) (layers "*.Cu" "*.Mask") (remove_unused_layers no) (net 6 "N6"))
  (pad "1" thru_hole circle (at 0 18.75 270) (size 3 3) (drill 1.2) (layers "*.Cu" "*.Mask") (remove_unused_layers no) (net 6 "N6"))
  (pad "2" thru_hole circle (at 0 -18.75 270) (size 3 3) (drill 1.2) (layers "*.Cu" "*.Mask") (remove_unused_layers no) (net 4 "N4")
   (zone_connect 2))
  (pad "2" thru_hole circle (at 0 -13.75 270) (size 3 3) (drill 1.2) (layers "*.Cu" "*.Mask") (remove_unused_layers no) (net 4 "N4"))
  (pad "2" thru_hole circle (at 0 -11.25 270) (size 3 3) (drill 1.2) (layers "*.Cu" "*.Mask") (remove_unused_layers no) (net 4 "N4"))
  (pad "2" thru_hole circle (at 0 -7.5 270) (size 3 3) (drill 1.2) (layers "*.Cu" "*.Mask") (remove_unused_layers no) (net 4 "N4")))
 (gr_line (start 45.0005 48.5) (end 245.0005 48.5) (stroke (width 0.05) (type default)) (layer "Edge.Cuts"))
 (gr_line (start 250.0005 53.5) (end 250.0005 140.5) (stroke (width 0.05) (type default)) (layer "Edge.Cuts"))
 (gr_line (start 250.0005 140.5) (end 245.0005 145.5) (stroke (width 0.05) (type default)) (layer "Edge.Cuts"))
 (gr_line (start 40.0005 53.5) (end 45.0005 48.5) (stroke (width 0.05) (type default)) (layer "Edge.Cuts"))
 (gr_line (start 245.0005 145.5) (end 45.0005 145.5) (stroke (width 0.05) (type default)) (layer "Edge.Cuts"))
 (gr_line (start 40.0005 140.5) (end 40.0005 53.5) (stroke (width 0.05) (type default)) (layer "Edge.Cuts"))
 (gr_line (start 245.0005 48.5) (end 250.0005 53.5) (stroke (width 0.05) (type default)) (layer "Edge.Cuts"))
 (gr_line (start 45.0005 145.5) (end 40.0005 140.5) (stroke (width 0.05) (type default)) (layer "Edge.Cuts"))
 (segment (start 65.5005 133.25) (end 50.0015 117.751) (width 19) (layer "F.Cu") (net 8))
 (segment (start 50.0015 117.751) (end 50.0015 75.749) (width 19) (layer "F.Cu") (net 8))
 (segment (start 50.0015 75.749) (end 65.5005 60.25) (width 19) (layer "F.Cu") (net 8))
 (segment (start 61.834833 109.083333) (end 50.0015 97.25) (width 19) (layer "F.Cu") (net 8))
 (segment (start 65.5005 109.083333) (end 61.834833 109.083333) (width 19) (layer "F.Cu") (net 8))
 (segment (start 62.834833 84.416667) (end 50.0015 97.25) (width 19) (layer "F.Cu") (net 8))
 (segment (start 65.5005 84.416667) (end 62.834833 84.416667) (width 19) (layer "F.Cu") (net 8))
 (segment (start 65.5005 84.416667) (end 62.834833 84.416667) (width 19) (layer "B.Cu") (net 8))
 (segment (start 65.5005 109.083333) (end 61.834833 109.083333) (width 19) (layer "B.Cu") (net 8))
 (segment (start 50.0015 117.751) (end 50.0015 75.749) (width 19) (layer "B.Cu") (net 8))
 (segment (start 62.834833 84.416667) (end 50.0015 97.25) (width 19) (layer "B.Cu") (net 8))
 (segment (start 65.5005 133.25) (end 50.0015 117.751) (width 19) (layer "B.Cu") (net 8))
 (segment (start 61.834833 109.083333) (end 50.0015 97.25) (width 19) (layer "B.Cu") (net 8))
 (segment (start 50.0015 75.749) (end 65.5005 60.25) (width 19) (layer "B.Cu") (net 8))
 (segment (start 93.0005 133.25) (end 109.2505 133.25) (width 19) (layer "F.Cu") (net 9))
 (segment (start 93.0005 133.25) (end 109.2505 133.25) (width 19) (layer "B.Cu") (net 9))
 (segment (start 136.7505 133.25) (end 153.0005 133.25) (width 19) (layer "F.Cu") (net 12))
 (segment (start 136.7505 133.25) (end 153.0005 133.25) (width 19) (layer "B.Cu") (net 12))
 (segment (start 180.5005 133.25) (end 197.0005 133.25) (width 19) (layer "F.Cu") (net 14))
 (segment (start 180.5005 133.25) (end 197.0005 133.25) (width 19) (layer "B.Cu") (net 14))
 (segment (start 227.666167 84.416667) (end 239.9995 96.75) (width 19) (layer "F.Cu") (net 4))
 (segment (start 224.5005 133.25) (end 239.9995 117.751) (width 19) (layer "F.Cu") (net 4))
 (segment (start 239.9995 117.751) (end 239.9995 75.749) (width 19) (layer "F.Cu") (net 4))
 (segment (start 224.5005 84.416667) (end 227.666167 84.416667) (width 19) (layer "F.Cu") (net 4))
 (segment (start 227.666167 109.083333) (end 239.9995 96.75) (width 19) (layer "F.Cu") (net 4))
 (segment (start 239.9995 75.749) (end 224.5005 60.25) (width 19) (layer "F.Cu") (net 4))
 (segment (start 224.5005 109.083333) (end 227.666167 109.083333) (width 19) (layer "F.Cu") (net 4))
 (segment (start 239.9995 117.751) (end 239.9995 75.749) (width 19) (layer "B.Cu") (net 4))
 (segment (start 224.5005 84.416667) (end 227.666167 84.416667) (width 19) (layer "B.Cu") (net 4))
 (segment (start 227.666167 109.083333) (end 239.9995 96.75) (width 19) (layer "B.Cu") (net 4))
 (segment (start 224.5005 133.25) (end 239.9995 117.751) (width 19) (layer "B.Cu") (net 4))
 (segment (start 227.666167 84.416667) (end 239.9995 96.75) (width 19) (layer "B.Cu") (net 4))
 (segment (start 239.9995 75.749) (end 224.5005 60.25) (width 19) (layer "B.Cu") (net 4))
 (segment (start 224.5005 109.083333) (end 227.666167 109.083333) (width 19) (layer "B.Cu") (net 4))
 (segment (start 93.0005 109.083333) (end 109.2505 109.083333) (width 19) (layer "F.Cu") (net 1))
 (segment (start 93.0005 109.083333) (end 109.2505 109.083333) (width 19) (layer "B.Cu") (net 1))
 (segment (start 136.7505 109.083333) (end 153.0005 109.083333) (width 19) (layer "F.Cu") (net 2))
 (segment (start 136.7505 109.083333) (end 153.0005 109.083333) (width 19) (layer "B.Cu") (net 2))
 (segment (start 180.5005 109.083333) (end 197.0005 109.083333) (width 19) (layer "F.Cu") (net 7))
 (segment (start 180.5005 109.083333) (end 197.0005 109.083333) (width 19) (layer "B.Cu") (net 7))
 (segment (start 93.0005 84.416667) (end 109.2505 84.416667) (width 19) (layer "F.Cu") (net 10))
 (segment (start 93.0005 84.416667) (end 109.2505 84.416667) (width 19) (layer "B.Cu") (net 10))
 (segment (start 136.7505 84.416667) (end 153.0005 84.416667) (width 19) (layer "F.Cu") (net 11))
 (segment (start 136.7505 84.416667) (end 153.0005 84.416667) (width 19) (layer "B.Cu") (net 11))
 (segment (start 180.5005 84.416667) (end 197.0005 84.416667) (width 19) (layer "F.Cu") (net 3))
 (segment (start 180.5005 84.416667) (end 197.0005 84.416667) (width 19) (layer "B.Cu") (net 3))
 (segment (start 93.0005 60.25) (end 109.2505 60.25) (width 19) (layer "F.Cu") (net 13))
 (segment (start 93.0005 60.25) (end 109.2505 60.25) (width 19) (layer "B.Cu") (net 13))
 (segment (start 136.7505 60.25) (end 153.0005 60.25) (width 19) (layer "F.Cu") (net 5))
 (segment (start 136.7505 60.25) (end 153.0005 60.25) (width 19) (layer "B.Cu") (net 5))
 (segment (start 180.5005 60.25) (end 197.0005 60.25) (width 19) (layer "F.Cu") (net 6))
 (segment (start 180.5005 60.25) (end 197.0005 60.25) (width 19) (layer "B.Cu") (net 6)))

